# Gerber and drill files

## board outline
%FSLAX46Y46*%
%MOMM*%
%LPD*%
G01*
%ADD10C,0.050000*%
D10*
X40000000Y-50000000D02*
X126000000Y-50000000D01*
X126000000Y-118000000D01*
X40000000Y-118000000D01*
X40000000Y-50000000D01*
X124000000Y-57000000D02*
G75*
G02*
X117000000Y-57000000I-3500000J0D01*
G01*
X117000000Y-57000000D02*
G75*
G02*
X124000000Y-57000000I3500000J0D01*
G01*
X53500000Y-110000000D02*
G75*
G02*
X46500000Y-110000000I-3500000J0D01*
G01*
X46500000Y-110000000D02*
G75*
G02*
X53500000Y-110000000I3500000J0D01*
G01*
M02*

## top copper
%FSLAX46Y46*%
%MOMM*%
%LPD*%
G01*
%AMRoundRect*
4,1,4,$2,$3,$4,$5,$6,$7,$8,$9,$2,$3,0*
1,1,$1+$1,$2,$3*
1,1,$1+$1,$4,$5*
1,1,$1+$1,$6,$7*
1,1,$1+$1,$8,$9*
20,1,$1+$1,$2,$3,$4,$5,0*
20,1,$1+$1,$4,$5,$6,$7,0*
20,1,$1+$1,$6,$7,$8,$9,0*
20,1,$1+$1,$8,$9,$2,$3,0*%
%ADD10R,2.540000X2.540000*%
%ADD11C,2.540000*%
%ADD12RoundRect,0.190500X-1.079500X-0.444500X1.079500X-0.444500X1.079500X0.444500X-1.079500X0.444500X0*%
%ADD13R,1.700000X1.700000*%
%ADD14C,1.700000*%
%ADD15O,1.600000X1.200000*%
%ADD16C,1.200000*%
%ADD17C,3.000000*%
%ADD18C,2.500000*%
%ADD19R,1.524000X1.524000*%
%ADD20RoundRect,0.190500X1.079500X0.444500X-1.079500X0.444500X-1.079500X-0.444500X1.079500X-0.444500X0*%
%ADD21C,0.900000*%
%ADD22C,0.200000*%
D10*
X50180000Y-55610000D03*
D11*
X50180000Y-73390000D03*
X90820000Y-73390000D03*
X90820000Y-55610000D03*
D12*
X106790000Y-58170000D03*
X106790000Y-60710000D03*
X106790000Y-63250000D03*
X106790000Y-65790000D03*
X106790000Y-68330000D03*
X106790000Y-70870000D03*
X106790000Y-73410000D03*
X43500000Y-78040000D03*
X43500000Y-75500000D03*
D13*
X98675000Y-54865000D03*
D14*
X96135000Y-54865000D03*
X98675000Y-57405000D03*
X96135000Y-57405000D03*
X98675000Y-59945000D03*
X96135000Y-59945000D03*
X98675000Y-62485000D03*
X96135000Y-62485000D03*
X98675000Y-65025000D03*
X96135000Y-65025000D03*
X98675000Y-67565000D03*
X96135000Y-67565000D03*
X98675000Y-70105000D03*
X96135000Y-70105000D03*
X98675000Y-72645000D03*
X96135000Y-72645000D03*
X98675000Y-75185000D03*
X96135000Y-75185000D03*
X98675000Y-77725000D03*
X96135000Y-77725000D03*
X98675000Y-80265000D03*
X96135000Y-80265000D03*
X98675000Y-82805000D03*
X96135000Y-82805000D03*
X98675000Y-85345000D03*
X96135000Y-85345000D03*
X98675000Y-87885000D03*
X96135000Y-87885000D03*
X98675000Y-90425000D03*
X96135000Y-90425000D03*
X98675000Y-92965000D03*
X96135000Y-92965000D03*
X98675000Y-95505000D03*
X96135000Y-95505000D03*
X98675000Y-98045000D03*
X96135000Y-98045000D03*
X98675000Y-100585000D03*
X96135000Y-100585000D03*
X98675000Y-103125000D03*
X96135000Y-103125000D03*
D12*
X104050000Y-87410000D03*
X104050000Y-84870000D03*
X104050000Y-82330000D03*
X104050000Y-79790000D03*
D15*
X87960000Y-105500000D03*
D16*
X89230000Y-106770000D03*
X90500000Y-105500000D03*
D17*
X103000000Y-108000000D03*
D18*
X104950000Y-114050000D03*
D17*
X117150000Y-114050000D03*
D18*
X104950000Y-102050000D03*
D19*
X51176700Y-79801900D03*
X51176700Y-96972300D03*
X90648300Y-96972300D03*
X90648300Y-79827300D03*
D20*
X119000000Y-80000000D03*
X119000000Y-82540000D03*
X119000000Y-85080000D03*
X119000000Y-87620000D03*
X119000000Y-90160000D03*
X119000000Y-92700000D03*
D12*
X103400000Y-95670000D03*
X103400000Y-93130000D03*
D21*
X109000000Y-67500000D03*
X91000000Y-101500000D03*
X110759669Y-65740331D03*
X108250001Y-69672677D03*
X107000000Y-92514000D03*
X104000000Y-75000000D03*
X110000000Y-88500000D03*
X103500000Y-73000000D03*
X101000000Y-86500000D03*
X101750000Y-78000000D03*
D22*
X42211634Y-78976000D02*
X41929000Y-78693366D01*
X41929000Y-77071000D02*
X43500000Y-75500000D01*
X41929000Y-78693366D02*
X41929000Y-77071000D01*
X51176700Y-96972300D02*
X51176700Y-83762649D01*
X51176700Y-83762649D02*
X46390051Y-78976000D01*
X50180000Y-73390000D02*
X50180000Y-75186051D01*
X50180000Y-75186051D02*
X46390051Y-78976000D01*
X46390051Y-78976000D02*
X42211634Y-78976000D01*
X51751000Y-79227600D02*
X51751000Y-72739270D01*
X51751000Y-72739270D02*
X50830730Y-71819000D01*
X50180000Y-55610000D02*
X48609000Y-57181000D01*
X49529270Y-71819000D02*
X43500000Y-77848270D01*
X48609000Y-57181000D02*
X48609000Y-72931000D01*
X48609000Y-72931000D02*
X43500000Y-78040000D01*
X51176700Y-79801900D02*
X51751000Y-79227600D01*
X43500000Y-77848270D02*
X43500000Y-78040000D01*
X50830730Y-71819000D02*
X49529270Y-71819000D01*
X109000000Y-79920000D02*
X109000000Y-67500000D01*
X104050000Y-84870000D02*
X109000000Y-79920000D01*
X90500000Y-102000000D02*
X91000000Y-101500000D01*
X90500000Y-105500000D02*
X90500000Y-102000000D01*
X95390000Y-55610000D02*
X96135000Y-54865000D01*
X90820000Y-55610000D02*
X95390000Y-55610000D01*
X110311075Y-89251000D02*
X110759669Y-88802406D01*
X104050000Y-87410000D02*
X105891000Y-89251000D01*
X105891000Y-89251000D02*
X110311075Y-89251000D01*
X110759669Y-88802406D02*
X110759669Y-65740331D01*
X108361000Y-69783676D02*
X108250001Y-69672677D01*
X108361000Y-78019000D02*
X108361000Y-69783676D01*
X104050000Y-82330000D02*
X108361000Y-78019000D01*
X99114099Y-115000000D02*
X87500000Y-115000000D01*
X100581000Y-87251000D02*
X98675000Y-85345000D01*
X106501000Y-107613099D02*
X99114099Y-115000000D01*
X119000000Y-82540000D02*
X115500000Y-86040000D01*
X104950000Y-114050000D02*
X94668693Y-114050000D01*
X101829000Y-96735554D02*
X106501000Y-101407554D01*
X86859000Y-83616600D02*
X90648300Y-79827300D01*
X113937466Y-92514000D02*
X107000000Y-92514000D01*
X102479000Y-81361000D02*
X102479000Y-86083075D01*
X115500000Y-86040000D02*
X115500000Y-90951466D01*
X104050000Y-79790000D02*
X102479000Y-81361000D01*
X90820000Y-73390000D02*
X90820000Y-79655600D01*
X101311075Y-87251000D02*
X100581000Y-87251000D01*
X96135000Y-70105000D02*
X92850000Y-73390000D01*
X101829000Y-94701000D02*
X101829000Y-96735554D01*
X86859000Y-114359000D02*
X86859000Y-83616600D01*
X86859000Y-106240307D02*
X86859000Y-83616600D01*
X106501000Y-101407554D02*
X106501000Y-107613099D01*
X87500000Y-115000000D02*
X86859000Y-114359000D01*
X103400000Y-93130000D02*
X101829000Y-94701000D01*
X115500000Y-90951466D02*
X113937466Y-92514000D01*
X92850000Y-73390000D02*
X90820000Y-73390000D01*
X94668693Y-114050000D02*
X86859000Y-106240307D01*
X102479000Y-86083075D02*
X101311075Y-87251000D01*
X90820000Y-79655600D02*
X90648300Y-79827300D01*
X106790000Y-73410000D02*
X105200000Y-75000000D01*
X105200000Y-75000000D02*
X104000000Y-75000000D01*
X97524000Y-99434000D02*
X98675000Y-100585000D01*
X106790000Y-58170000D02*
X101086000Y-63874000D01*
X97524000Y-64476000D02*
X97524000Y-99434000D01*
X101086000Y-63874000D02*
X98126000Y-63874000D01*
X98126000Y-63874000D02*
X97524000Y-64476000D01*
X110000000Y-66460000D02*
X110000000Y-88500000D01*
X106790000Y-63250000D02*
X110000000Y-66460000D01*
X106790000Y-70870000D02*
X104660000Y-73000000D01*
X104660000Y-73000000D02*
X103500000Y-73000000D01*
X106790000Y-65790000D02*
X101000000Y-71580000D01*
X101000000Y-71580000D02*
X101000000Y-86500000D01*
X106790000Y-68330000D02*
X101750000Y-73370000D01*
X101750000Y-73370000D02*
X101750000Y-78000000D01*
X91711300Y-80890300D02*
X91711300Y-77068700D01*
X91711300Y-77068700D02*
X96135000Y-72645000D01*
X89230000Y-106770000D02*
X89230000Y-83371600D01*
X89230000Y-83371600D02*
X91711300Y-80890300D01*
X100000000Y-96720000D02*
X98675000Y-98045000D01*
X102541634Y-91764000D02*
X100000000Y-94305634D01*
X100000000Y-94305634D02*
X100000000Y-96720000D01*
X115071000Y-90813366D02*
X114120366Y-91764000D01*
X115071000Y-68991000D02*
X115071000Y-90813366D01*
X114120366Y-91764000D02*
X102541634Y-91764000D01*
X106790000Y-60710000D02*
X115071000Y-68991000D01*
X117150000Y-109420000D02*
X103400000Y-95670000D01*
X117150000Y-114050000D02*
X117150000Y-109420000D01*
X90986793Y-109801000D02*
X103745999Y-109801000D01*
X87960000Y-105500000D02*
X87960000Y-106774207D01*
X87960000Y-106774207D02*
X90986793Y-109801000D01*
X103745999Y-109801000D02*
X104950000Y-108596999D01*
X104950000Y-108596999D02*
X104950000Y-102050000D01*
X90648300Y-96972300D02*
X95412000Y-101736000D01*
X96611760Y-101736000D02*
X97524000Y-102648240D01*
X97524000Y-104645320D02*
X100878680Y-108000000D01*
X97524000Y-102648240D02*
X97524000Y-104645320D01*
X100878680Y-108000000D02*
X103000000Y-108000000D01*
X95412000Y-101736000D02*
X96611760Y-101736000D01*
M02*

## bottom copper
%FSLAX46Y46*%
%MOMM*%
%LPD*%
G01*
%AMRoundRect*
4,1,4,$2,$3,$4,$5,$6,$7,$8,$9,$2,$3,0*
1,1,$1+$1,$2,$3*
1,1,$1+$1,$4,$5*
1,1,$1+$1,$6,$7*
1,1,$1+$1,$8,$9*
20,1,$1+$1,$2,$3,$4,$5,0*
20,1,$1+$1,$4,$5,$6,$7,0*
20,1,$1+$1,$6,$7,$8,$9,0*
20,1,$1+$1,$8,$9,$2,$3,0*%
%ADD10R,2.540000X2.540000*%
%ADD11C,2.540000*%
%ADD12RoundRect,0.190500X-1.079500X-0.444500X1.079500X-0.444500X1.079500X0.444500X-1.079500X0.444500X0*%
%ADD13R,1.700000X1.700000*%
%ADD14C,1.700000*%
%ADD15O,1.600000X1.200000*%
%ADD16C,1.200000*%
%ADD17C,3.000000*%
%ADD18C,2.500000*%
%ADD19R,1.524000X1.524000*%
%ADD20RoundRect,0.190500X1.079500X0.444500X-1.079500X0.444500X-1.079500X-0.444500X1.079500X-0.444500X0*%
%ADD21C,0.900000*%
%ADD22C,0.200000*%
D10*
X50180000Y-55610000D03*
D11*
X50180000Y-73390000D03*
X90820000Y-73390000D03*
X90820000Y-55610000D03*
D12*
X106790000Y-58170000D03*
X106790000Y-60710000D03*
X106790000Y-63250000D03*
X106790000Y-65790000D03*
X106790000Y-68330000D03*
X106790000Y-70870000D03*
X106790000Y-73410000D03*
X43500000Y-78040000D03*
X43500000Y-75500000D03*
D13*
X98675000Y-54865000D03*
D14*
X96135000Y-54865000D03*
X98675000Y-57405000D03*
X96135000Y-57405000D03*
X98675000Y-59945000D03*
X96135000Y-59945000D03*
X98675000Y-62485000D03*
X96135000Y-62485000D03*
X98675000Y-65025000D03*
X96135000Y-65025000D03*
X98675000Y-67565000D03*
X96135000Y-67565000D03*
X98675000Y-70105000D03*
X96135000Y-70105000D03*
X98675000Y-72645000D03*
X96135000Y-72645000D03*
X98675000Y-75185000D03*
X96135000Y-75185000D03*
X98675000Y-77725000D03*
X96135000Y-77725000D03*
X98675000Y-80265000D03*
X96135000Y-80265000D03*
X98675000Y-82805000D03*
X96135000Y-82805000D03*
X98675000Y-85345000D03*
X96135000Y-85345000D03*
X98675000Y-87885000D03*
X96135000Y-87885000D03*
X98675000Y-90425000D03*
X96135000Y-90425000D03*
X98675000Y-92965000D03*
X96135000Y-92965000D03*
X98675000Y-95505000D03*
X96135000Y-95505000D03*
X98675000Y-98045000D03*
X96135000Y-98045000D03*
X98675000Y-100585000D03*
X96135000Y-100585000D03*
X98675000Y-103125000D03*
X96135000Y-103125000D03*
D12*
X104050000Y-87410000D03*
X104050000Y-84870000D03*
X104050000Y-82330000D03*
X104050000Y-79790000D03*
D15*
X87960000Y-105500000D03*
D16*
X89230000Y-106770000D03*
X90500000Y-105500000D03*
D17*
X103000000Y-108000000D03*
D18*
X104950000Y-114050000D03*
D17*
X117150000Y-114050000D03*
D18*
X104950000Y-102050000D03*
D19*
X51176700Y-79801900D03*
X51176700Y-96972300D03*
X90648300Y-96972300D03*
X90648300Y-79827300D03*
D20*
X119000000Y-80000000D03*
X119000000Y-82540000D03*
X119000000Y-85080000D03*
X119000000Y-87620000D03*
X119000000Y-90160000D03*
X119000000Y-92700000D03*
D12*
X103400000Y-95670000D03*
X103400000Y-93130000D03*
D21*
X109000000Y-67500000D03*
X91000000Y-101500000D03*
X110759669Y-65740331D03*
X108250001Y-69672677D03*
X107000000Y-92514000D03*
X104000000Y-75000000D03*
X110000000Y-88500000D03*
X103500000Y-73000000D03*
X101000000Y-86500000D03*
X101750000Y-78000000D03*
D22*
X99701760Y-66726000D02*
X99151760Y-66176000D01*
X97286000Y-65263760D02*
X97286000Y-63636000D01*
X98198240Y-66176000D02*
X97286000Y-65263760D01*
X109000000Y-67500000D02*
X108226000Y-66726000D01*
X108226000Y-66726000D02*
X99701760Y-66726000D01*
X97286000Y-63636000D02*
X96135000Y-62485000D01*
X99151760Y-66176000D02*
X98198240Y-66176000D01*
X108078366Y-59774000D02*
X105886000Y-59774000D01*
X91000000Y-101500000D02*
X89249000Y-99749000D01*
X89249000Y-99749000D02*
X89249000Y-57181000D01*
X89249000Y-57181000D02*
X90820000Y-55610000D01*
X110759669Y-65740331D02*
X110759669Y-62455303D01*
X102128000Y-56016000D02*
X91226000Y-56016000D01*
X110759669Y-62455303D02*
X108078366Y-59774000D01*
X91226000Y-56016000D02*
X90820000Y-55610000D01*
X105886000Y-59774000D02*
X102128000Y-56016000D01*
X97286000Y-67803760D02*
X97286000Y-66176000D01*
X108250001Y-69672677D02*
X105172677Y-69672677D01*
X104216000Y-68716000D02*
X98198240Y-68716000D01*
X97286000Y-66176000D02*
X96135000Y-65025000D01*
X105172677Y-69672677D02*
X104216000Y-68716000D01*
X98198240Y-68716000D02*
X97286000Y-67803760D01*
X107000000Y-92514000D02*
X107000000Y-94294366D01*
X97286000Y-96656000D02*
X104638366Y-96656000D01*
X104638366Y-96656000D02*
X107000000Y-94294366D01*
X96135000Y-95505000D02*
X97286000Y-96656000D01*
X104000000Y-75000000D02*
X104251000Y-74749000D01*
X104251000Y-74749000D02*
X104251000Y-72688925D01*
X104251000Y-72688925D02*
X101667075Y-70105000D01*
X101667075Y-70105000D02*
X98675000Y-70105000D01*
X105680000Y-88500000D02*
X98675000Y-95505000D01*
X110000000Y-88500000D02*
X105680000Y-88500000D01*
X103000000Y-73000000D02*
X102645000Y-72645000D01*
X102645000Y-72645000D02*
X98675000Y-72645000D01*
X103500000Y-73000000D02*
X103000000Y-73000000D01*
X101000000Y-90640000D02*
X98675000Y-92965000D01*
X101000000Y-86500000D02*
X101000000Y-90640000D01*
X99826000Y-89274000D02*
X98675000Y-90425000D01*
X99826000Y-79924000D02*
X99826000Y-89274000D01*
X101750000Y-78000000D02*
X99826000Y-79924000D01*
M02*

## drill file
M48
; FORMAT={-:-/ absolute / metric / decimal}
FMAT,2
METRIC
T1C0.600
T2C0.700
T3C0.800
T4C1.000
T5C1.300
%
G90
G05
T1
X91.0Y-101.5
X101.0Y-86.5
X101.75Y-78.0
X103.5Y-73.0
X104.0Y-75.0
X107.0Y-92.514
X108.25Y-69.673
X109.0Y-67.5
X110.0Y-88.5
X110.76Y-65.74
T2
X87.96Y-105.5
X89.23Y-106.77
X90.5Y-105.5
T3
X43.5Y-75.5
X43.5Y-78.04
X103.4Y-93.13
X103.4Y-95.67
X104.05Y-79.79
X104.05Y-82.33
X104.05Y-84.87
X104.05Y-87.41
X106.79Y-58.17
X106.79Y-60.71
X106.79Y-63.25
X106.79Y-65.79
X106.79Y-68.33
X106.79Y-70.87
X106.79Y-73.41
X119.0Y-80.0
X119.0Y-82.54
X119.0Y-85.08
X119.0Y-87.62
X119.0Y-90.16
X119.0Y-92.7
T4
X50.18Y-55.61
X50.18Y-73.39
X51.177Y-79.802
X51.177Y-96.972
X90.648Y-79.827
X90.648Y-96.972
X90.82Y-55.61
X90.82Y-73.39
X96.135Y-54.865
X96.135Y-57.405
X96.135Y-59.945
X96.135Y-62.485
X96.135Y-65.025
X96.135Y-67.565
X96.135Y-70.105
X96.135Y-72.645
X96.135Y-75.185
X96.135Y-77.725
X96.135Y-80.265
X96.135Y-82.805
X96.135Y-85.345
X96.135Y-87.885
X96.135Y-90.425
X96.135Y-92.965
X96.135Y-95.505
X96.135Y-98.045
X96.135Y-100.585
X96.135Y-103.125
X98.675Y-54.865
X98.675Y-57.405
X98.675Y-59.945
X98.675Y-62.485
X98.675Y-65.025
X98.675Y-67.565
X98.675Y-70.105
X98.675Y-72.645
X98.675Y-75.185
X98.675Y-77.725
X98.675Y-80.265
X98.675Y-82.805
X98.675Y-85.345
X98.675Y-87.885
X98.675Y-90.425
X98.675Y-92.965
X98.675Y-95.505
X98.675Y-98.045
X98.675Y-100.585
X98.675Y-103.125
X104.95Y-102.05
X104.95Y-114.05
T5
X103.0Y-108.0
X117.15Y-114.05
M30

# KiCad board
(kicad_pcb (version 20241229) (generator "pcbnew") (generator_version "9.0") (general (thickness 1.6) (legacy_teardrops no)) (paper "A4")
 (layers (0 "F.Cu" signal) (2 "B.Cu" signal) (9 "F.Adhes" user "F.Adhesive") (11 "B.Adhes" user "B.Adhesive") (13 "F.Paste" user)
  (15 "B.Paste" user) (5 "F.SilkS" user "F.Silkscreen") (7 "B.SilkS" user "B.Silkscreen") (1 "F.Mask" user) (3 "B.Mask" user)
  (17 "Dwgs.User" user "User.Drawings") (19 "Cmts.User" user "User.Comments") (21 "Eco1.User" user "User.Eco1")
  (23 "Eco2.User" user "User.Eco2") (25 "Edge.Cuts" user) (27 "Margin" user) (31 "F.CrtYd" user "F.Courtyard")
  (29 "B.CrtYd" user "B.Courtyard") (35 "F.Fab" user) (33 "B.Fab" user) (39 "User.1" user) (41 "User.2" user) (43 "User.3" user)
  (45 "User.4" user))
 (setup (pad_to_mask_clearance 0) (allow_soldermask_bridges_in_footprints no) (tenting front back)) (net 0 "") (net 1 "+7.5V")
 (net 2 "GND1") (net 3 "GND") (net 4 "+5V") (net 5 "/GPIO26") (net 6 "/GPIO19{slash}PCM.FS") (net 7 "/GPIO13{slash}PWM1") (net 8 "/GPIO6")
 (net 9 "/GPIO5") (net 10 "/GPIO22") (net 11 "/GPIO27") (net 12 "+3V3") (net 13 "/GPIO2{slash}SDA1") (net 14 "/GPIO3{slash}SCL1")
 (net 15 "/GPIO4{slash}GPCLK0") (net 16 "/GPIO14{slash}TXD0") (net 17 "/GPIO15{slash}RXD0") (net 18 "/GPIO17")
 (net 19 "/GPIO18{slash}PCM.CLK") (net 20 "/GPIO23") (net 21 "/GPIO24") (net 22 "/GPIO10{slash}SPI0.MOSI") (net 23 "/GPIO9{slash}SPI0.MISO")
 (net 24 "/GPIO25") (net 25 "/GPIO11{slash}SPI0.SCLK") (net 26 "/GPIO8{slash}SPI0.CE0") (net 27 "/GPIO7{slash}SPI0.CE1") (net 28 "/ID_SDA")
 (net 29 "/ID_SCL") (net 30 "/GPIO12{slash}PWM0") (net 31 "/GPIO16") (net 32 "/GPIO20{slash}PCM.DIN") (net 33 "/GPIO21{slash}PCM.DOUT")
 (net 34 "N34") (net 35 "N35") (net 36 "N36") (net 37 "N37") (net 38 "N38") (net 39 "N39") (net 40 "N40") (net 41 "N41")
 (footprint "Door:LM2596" (layer "F.Cu") (at 50.18 55.61)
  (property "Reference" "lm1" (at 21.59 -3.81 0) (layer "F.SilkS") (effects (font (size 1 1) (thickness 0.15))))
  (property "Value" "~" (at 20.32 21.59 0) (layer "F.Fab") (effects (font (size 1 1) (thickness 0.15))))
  (pad "1" thru_hole rect (at 0 0) (size 2.54 2.54) (drill 1) (layers "*.Cu" "*.Mask") (remove_unused_layers no) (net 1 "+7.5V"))
  (pad "2" thru_hole circle (at 0 17.78) (size 2.54 2.54) (drill 1) (layers "*.Cu" "*.Mask") (remove_unused_layers no) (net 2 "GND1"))
  (pad "3" thru_hole circle (at 40.64 17.78) (size 2.54 2.54) (drill 1) (layers "*.Cu" "*.Mask") (remove_unused_layers no) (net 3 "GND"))
  (pad "4" thru_hole circle (at 40.64 0) (size 2.54 2.54) (drill 1) (layers "*.Cu" "*.Mask") (remove_unused_layers no) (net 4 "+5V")))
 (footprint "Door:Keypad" (layer "F.Cu") (at 101.71 75.95)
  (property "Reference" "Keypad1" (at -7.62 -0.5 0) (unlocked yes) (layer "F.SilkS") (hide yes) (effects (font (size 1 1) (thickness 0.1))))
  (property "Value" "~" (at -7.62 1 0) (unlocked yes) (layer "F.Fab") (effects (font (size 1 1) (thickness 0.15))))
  (pad "2" thru_hole roundrect (at 5.08 -17.78) (size 2.54 1.27) (drill 0.8) (layers "*.Cu" "*.Mask") (remove_unused_layers no)
   (roundrect_rratio 0.15) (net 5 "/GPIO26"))
  (pad "3" thru_hole roundrect (at 5.08 -15.24) (size 2.54 1.27) (drill 0.8) (layers "*.Cu" "*.Mask") (remove_unused_layers no)
   (roundrect_rratio 0.15) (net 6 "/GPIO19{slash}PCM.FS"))
  (pad "4" thru_hole roundrect (at 5.08 -12.7) (size 2.54 1.27) (drill 0.8) (layers "*.Cu" "*.Mask") (remove_unused_layers no)
   (roundrect_rratio 0.15) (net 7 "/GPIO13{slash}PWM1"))
  (pad "5" thru_hole roundrect (at 5.08 -10.16) (size 2.54 1.27) (drill 0.8) (layers "*.Cu" "*.Mask") (remove_unused_layers no)
   (roundrect_rratio 0.15) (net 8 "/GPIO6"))
  (pad "6" thru_hole roundrect (at 5.08 -7.62) (size 2.54 1.27) (drill 0.8) (layers "*.Cu" "*.Mask") (remove_unused_layers no)
   (roundrect_rratio 0.15) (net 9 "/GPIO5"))
  (pad "7" thru_hole roundrect (at 5.08 -5.08) (size 2.54 1.27) (drill 0.8) (layers "*.Cu" "*.Mask") (remove_unused_layers no)
   (roundrect_rratio 0.15) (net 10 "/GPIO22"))
  (pad "8" thru_hole roundrect (at 5.08 -2.54) (size 2.54 1.27) (drill 0.8) (layers "*.Cu" "*.Mask") (remove_unused_layers no)
   (roundrect_rratio 0.15) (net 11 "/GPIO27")))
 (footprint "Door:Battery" (layer "F.Cu") (at 48.58 83.12)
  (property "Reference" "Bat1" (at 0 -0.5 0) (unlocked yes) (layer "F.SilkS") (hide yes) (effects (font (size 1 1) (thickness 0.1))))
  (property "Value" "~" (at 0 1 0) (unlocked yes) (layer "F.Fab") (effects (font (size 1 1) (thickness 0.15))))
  (pad "1" thru_hole roundrect (at -5.08 -5.08) (size 2.54 1.27) (drill 0.8) (layers "*.Cu" "*.Mask") (remove_unused_layers no)
   (roundrect_rratio 0.15) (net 1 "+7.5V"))
  (pad "2" thru_hole roundrect (at -5.08 -7.62) (size 2.54 1.27) (drill 0.8) (layers "*.Cu" "*.Mask") (remove_unused_layers no)
   (roundrect_rratio 0.15) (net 2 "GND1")))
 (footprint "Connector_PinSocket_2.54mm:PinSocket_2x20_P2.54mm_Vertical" (layer "F.Cu") (at 98.675 54.865)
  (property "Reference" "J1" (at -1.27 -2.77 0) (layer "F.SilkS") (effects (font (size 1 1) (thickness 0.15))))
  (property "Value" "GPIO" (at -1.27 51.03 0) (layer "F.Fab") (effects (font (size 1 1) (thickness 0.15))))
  (pad "1" thru_hole rect (at 0 0) (size 1.7 1.7) (drill 1) (layers "*.Cu" "*.Mask") (remove_unused_layers no) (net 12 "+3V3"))
  (pad "2" thru_hole circle (at -2.54 0) (size 1.7 1.7) (drill 1) (layers "*.Cu" "*.Mask") (remove_unused_layers no) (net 4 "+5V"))
  (pad "3" thru_hole circle (at 0 2.54) (size 1.7 1.7) (drill 1) (layers "*.Cu" "*.Mask") (remove_unused_layers no)
   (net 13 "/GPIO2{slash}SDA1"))
  (pad "4" thru_hole circle (at -2.54 2.54) (size 1.7 1.7) (drill 1) (layers "*.Cu" "*.Mask") (remove_unused_layers no) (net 4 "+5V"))
  (pad "5" thru_hole circle (at 0 5.08) (size 1.7 1.7) (drill 1) (layers "*.Cu" "*.Mask") (remove_unused_layers no)
   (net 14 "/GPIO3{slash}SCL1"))
  (pad "6" thru_hole circle (at -2.54 5.08) (size 1.7 1.7) (drill 1) (layers "*.Cu" "*.Mask") (remove_unused_layers no) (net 3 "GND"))
  (pad "7" thru_hole circle (at 0 7.62) (size 1.7 1.7) (drill 1) (layers "*.Cu" "*.Mask") (remove_unused_layers no)
   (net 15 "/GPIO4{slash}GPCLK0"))
  (pad "8" thru_hole circle (at -2.54 7.62) (size 1.7 1.7) (drill 1) (layers "*.Cu" "*.Mask") (remove_unused_layers no)
   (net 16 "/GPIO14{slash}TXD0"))
  (pad "9" thru_hole circle (at 0 10.16) (size 1.7 1.7) (drill 1) (layers "*.Cu" "*.Mask") (remove_unused_layers no) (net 3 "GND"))
  (pad "10" thru_hole circle (at -2.54 10.16) (size 1.7 1.7) (drill 1) (layers "*.Cu" "*.Mask") (remove_unused_layers no)
   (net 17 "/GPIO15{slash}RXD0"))
  (pad "11" thru_hole circle (at 0 12.7) (size 1.7 1.7) (drill 1) (layers "*.Cu" "*.Mask") (remove_unused_layers no) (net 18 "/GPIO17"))
  (pad "12" thru_hole circle (at -2.54 12.7) (size 1.7 1.7) (drill 1) (layers "*.Cu" "*.Mask") (remove_unused_layers no)
   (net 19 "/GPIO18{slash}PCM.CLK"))
  (pad "13" thru_hole circle (at 0 15.24) (size 1.7 1.7) (drill 1) (layers "*.Cu" "*.Mask") (remove_unused_layers no) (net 11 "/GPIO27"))
  (pad "14" thru_hole circle (at -2.54 15.24) (size 1.7 1.7) (drill 1) (layers "*.Cu" "*.Mask") (remove_unused_layers no) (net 3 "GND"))
  (pad "15" thru_hole circle (at 0 17.78) (size 1.7 1.7) (drill 1) (layers "*.Cu" "*.Mask") (remove_unused_layers no) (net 10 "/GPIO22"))
  (pad "16" thru_hole circle (at -2.54 17.78) (size 1.7 1.7) (drill 1) (layers "*.Cu" "*.Mask") (remove_unused_layers no) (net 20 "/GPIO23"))
  (pad "17" thru_hole circle (at 0 20.32) (size 1.7 1.7) (drill 1) (layers "*.Cu" "*.Mask") (remove_unused_layers no) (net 12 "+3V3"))
  (pad "18" thru_hole circle (at -2.54 20.32) (size 1.7 1.7) (drill 1) (layers "*.Cu" "*.Mask") (remove_unused_layers no) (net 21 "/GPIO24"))
  (pad "19" thru_hole circle (at 0 22.86) (size 1.7 1.7) (drill 1) (layers "*.Cu" "*.Mask") (remove_unused_layers no)
   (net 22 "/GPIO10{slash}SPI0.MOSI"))
  (pad "20" thru_hole circle (at -2.54 22.86) (size 1.7 1.7) (drill 1) (layers "*.Cu" "*.Mask") (remove_unused_layers no) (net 3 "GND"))
  (pad "21" thru_hole circle (at 0 25.4) (size 1.7 1.7) (drill 1) (layers "*.Cu" "*.Mask") (remove_unused_layers no)
   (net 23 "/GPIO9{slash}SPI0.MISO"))
  (pad "22" thru_hole circle (at -2.54 25.4) (size 1.7 1.7) (drill 1) (layers "*.Cu" "*.Mask") (remove_unused_layers no) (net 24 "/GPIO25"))
  (pad "23" thru_hole circle (at 0 27.94) (size 1.7 1.7) (drill 1) (layers "*.Cu" "*.Mask") (remove_unused_layers no)
   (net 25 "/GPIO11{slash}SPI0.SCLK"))
  (pad "24" thru_hole circle (at -2.54 27.94) (size 1.7 1.7) (drill 1) (layers "*.Cu" "*.Mask") (remove_unused_layers no)
   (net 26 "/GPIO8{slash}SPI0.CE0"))
  (pad "25" thru_hole circle (at 0 30.48) (size 1.7 1.7) (drill 1) (layers "*.Cu" "*.Mask") (remove_unused_layers no) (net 3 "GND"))
  (pad "26" thru_hole circle (at -2.54 30.48) (size 1.7 1.7) (drill 1) (layers "*.Cu" "*.Mask") (remove_unused_layers no)
   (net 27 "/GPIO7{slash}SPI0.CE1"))
  (pad "27" thru_hole circle (at 0 33.02) (size 1.7 1.7) (drill 1) (layers "*.Cu" "*.Mask") (remove_unused_layers no) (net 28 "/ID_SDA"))
  (pad "28" thru_hole circle (at -2.54 33.02) (size 1.7 1.7) (drill 1) (layers "*.Cu" "*.Mask") (remove_unused_layers no) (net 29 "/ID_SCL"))
  (pad "29" thru_hole circle (at 0 35.56) (size 1.7 1.7) (drill 1) (layers "*.Cu" "*.Mask") (remove_unused_layers no) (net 9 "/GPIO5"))
  (pad "30" thru_hole circle (at -2.54 35.56) (size 1.7 1.7) (drill 1) (layers "*.Cu" "*.Mask") (remove_unused_layers no) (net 3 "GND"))
  (pad "31" thru_hole circle (at 0 38.1) (size 1.7 1.7) (drill 1) (layers "*.Cu" "*.Mask") (remove_unused_layers no) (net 8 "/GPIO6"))
  (pad "32" thru_hole circle (at -2.54 38.1) (size 1.7 1.7) (drill 1) (layers "*.Cu" "*.Mask") (remove_unused_layers no)
   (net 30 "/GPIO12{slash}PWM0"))
  (pad "33" thru_hole circle (at 0 40.64) (size 1.7 1.7) (drill 1) (layers "*.Cu" "*.Mask") (remove_unused_layers no)
   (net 7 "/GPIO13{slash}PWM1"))
  (pad "34" thru_hole circle (at -2.54 40.64) (size 1.7 1.7) (drill 1) (layers "*.Cu" "*.Mask") (remove_unused_layers no) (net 3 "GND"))
  (pad "35" thru_hole circle (at 0 43.18) (size 1.7 1.7) (drill 1) (layers "*.Cu" "*.Mask") (remove_unused_layers no)
   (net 6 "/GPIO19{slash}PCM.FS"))
  (pad "36" thru_hole circle (at -2.54 43.18) (size 1.7 1.7) (drill 1) (layers "*.Cu" "*.Mask") (remove_unused_layers no) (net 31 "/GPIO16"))
  (pad "37" thru_hole circle (at 0 45.72) (size 1.7 1.7) (drill 1) (layers "*.Cu" "*.Mask") (remove_unused_layers no) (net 5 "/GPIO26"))
  (pad "38" thru_hole circle (at -2.54 45.72) (size 1.7 1.7) (drill 1) (layers "*.Cu" "*.Mask") (remove_unused_layers no)
   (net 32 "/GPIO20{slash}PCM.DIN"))
  (pad "39" thru_hole circle (at 0 48.26) (size 1.7 1.7) (drill 1) (layers "*.Cu" "*.Mask") (remove_unused_layers no) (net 3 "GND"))
  (pad "40" thru_hole circle (at -2.54 48.26) (size 1.7 1.7) (drill 1) (layers "*.Cu" "*.Mask") (remove_unused_layers no)
   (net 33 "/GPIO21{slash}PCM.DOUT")))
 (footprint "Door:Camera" (layer "F.Cu") (at 106.59 97.57)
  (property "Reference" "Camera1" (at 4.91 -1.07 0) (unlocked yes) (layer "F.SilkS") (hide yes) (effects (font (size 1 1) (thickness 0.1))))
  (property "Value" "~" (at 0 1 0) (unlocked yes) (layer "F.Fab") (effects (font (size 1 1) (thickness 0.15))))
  (pad "1" thru_hole roundrect (at -2.54 -10.16) (size 2.54 1.27) (drill 0.8) (layers "*.Cu" "*.Mask") (remove_unused_layers no)
   (roundrect_rratio 0.15) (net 4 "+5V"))
  (pad "2" thru_hole roundrect (at -2.54 -12.7) (size 2.54 1.27) (drill 0.8) (layers "*.Cu" "*.Mask") (remove_unused_layers no)
   (roundrect_rratio 0.15) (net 16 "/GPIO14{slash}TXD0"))
  (pad "3" thru_hole roundrect (at -2.54 -15.24) (size 2.54 1.27) (drill 0.8) (layers "*.Cu" "*.Mask") (remove_unused_layers no)
   (roundrect_rratio 0.15) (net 17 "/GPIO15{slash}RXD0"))
  (pad "4" thru_hole roundrect (at -2.54 -17.78) (size 2.54 1.27) (drill 0.8) (layers "*.Cu" "*.Mask") (remove_unused_layers no)
   (roundrect_rratio 0.15) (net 3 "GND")))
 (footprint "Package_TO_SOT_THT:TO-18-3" (layer "F.Cu") (at 87.96 105.5)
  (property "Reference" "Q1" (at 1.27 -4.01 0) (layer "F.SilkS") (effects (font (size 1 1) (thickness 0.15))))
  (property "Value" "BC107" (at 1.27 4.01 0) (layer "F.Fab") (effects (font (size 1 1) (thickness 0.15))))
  (pad "1" thru_hole oval (at 0 0) (size 1.6 1.2) (drill 0.7) (layers "*.Cu" "*.Mask") (remove_unused_layers no) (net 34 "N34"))
  (pad "2" thru_hole circle (at 1.27 1.27) (size 1.2 1.2) (drill 0.7) (layers "*.Cu" "*.Mask") (remove_unused_layers no) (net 20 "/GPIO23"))
  (pad "3" thru_hole circle (at 2.54 0) (size 1.2 1.2) (drill 0.7) (layers "*.Cu" "*.Mask") (remove_unused_layers no) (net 4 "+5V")))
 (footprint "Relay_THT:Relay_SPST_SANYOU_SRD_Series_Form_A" (layer "F.Cu") (at 103 108)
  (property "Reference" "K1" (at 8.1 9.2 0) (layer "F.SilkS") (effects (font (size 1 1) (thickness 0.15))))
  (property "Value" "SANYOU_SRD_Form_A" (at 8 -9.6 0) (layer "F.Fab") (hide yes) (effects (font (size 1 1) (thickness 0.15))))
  (pad "1" thru_hole circle (at 0 0 90) (size 3 3) (drill 1.3) (layers "*.Cu" "*.Mask") (remove_unused_layers no) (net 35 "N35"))
  (pad "2" thru_hole circle (at 1.95 6.05 90) (size 2.5 2.5) (drill 1) (layers "*.Cu" "*.Mask") (remove_unused_layers no) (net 3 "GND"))
  (pad "3" thru_hole circle (at 14.15 6.05 90) (size 3 3) (drill 1.3) (layers "*.Cu" "*.Mask") (remove_unused_layers no) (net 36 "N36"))
  (pad "5" thru_hole circle (at 1.95 -5.95 90) (size 2.5 2.5) (drill 1) (layers "*.Cu" "*.Mask") (remove_unused_layers no) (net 34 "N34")))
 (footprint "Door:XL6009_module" (layer "F.Cu") (at 92.5025 98.9535)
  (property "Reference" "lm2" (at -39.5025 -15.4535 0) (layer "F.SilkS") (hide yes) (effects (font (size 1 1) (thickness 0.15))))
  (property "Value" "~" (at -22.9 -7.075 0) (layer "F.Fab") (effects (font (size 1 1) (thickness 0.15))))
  (pad "1" thru_hole rect (at -41.3258 -19.1516) (size 1.524 1.524) (drill 1) (layers "*.Cu" "*.Mask") (remove_unused_layers no)
   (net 1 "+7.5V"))
  (pad "2" thru_hole rect (at -41.3258 -1.9812) (size 1.524 1.524) (drill 1) (layers "*.Cu" "*.Mask") (remove_unused_layers no)
   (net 2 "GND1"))
  (pad "3" thru_hole rect (at -1.8542 -1.9812) (size 1.524 1.524) (drill 1) (layers "*.Cu" "*.Mask") (remove_unused_layers no)
   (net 35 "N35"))
  (pad "4" thru_hole rect (at -1.8542 -19.1262) (size 1.524 1.524) (drill 1) (layers "*.Cu" "*.Mask") (remove_unused_layers no)
   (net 3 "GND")))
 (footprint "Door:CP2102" (layer "F.Cu") (at 116.46 77.46 180)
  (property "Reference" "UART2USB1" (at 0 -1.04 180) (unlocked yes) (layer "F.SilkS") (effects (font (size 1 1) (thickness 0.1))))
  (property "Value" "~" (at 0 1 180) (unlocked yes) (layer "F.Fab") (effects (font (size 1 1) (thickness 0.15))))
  (pad "1" thru_hole roundrect (at -2.54 -2.54 180) (size 2.54 1.27) (drill 0.8) (layers "*.Cu" "*.Mask") (remove_unused_layers no)
   (roundrect_rratio 0.15) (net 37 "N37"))
  (pad "2" thru_hole roundrect (at -2.54 -5.08 180) (size 2.54 1.27) (drill 0.8) (layers "*.Cu" "*.Mask") (remove_unused_layers no)
   (roundrect_rratio 0.15) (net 3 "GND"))
  (pad "3" thru_hole roundrect (at -2.54 -7.62 180) (size 2.54 1.27) (drill 0.8) (layers "*.Cu" "*.Mask") (remove_unused_layers no)
   (roundrect_rratio 0.15) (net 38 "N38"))
  (pad "4" thru_hole roundrect (at -2.54 -10.16 180) (size 2.54 1.27) (drill 0.8) (layers "*.Cu" "*.Mask") (remove_unused_layers no)
   (roundrect_rratio 0.15) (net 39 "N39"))
  (pad "5" thru_hole roundrect (at -2.54 -12.7 180) (size 2.54 1.27) (drill 0.8) (layers "*.Cu" "*.Mask") (remove_unused_layers no)
   (roundrect_rratio 0.15) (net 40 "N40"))
  (pad "6" thru_hole roundrect (at -2.54 -15.24 180) (size 2.54 1.27) (drill 0.8) (layers "*.Cu" "*.Mask") (remove_unused_layers no)
   (roundrect_rratio 0.15) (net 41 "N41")))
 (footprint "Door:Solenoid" (layer "F.Cu") (at 105.94 98.21)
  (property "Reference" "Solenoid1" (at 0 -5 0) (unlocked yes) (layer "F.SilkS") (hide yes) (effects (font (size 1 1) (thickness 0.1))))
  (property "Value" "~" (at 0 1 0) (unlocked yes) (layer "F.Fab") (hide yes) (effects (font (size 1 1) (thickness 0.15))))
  (pad "1" thru_hole roundrect (at -2.54 -2.54) (size 2.54 1.27) (drill 0.8) (layers "*.Cu" "*.Mask") (remove_unused_layers no)
   (roundrect_rratio 0.15) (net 36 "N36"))
  (pad "2" thru_hole roundrect (at -2.54 -5.08) (size 2.54 1.27) (drill 0.8) (layers "*.Cu" "*.Mask") (remove_unused_layers no)
   (roundrect_rratio 0.15) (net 3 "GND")))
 (gr_rect (start 40 50) (end 126 118) (stroke (width 0.05) (type default)) (fill no) (layer "Edge.Cuts"))
 (gr_circle (center 120.5 57) (end 124 57) (stroke (width 0.05) (type default)) (fill no) (layer "Edge.Cuts"))
 (gr_circle (center 50 110) (end 53.5 110) (stroke (width 0.05) (type default)) (fill no) (layer "Edge.Cuts"))
 (segment (start 42.211634 78.976) (end 41.929 78.693366) (width 0.2) (layer "F.Cu") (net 2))
 (segment (start 41.929 77.071) (end 43.5 75.5) (width 0.2) (layer "F.Cu") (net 2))
 (segment (start 41.929 78.693366) (end 41.929 77.071) (width 0.2) (layer "F.Cu") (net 2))
 (segment (start 51.1767 96.9723) (end 51.1767 83.762649) (width 0.2) (layer "F.Cu") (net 2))
 (segment (start 51.1767 83.762649) (end 46.390051 78.976) (width 0.2) (layer "F.Cu") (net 2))
 (segment (start 50.18 73.39) (end 50.18 75.186051) (width 0.2) (layer "F.Cu") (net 2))
 (segment (start 50.18 75.186051) (end 46.390051 78.976) (width 0.2) (layer "F.Cu") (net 2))
 (segment (start 46.390051 78.976) (end 42.211634 78.976) (width 0.2) (layer "F.Cu") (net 2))
 (segment (start 51.751 79.2276) (end 51.751 72.73927) (width 0.2) (layer "F.Cu") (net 1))
 (segment (start 51.751 72.73927) (end 50.83073 71.819) (width 0.2) (layer "F.Cu") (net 1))
 (segment (start 50.18 55.61) (end 48.609 57.181) (width 0.2) (layer "F.Cu") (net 1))
 (segment (start 49.52927 71.819) (end 43.5 77.84827) (width 0.2) (layer "F.Cu") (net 1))
 (segment (start 48.609 57.181) (end 48.609 72.931) (width 0.2) (layer "F.Cu") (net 1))
 (segment (start 48.609 72.931) (end 43.5 78.04) (width 0.2) (layer "F.Cu") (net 1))
 (segment (start 51.1767 79.8019) (end 51.751 79.2276) (width 0.2) (layer "F.Cu") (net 1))
 (segment (start 43.5 77.84827) (end 43.5 78.04) (width 0.2) (layer "F.Cu") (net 1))
 (segment (start 50.83073 71.819) (end 49.52927 71.819) (width 0.2) (layer "F.Cu") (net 1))
 (segment (start 109 79.92) (end 109 67.5) (width 0.2) (layer "F.Cu") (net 16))
 (segment (start 104.05 84.87) (end 109 79.92) (width 0.2) (layer "F.Cu") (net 16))
 (via (at 109 67.5) (size 0.9) (drill 0.6) (layers "F.Cu" "B.Cu") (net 16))
 (segment (start 99.70176 66.726) (end 99.15176 66.176) (width 0.2) (layer "B.Cu") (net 16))
 (segment (start 97.286 65.26376) (end 97.286 63.636) (width 0.2) (layer "B.Cu") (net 16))
 (segment (start 98.19824 66.176) (end 97.286 65.26376) (width 0.2) (layer "B.Cu") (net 16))
 (segment (start 109 67.5) (end 108.226 66.726) (width 0.2) (layer "B.Cu") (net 16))
 (segment (start 108.226 66.726) (end 99.70176 66.726) (width 0.2) (layer "B.Cu") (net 16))
 (segment (start 97.286 63.636) (end 96.135 62.485) (width 0.2) (layer "B.Cu") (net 16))
 (segment (start 99.15176 66.176) (end 98.19824 66.176) (width 0.2) (layer "B.Cu") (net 16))
 (segment (start 90.5 102) (end 91 101.5) (width 0.2) (layer "F.Cu") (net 4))
 (segment (start 90.5 105.5) (end 90.5 102) (width 0.2) (layer "F.Cu") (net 4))
 (segment (start 95.39 55.61) (end 96.135 54.865) (width 0.2) (layer "F.Cu") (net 4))
 (segment (start 90.82 55.61) (end 95.39 55.61) (width 0.2) (layer "F.Cu") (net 4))
 (segment (start 110.311075 89.251) (end 110.759669 88.802406) (width 0.2) (layer "F.Cu") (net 4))
 (segment (start 104.05 87.41) (end 105.891 89.251) (width 0.2) (layer "F.Cu") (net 4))
 (segment (start 105.891 89.251) (end 110.311075 89.251) (width 0.2) (layer "F.Cu") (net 4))
 (segment (start 110.759669 88.802406) (end 110.759669 65.740331) (width 0.2) (layer "F.Cu") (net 4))
 (via (at 91 101.5) (size 0.9) (drill 0.6) (layers "F.Cu" "B.Cu") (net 4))
 (via (at 110.759669 65.740331) (size 0.9) (drill 0.6) (layers "F.Cu" "B.Cu") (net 4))
 (segment (start 108.078366 59.774) (end 105.886 59.774) (width 0.2) (layer "B.Cu") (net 4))
 (segment (start 91 101.5) (end 89.249 99.749) (width 0.2) (layer "B.Cu") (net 4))
 (segment (start 89.249 99.749) (end 89.249 57.181) (width 0.2) (layer "B.Cu") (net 4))
 (segment (start 89.249 57.181) (end 90.82 55.61) (width 0.2) (layer "B.Cu") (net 4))
 (segment (start 110.759669 65.740331) (end 110.759669 62.455303) (width 0.2) (layer "B.Cu") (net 4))
 (segment (start 102.128 56.016) (end 91.226 56.016) (width 0.2) (layer "B.Cu") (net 4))
 (segment (start 110.759669 62.455303) (end 108.078366 59.774) (width 0.2) (layer "B.Cu") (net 4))
 (segment (start 91.226 56.016) (end 90.82 55.61) (width 0.2) (layer "B.Cu") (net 4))
 (segment (start 105.886 59.774) (end 102.128 56.016) (width 0.2) (layer "B.Cu") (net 4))
 (segment (start 108.361 69.783676) (end 108.250001 69.672677) (width 0.2) (layer "F.Cu") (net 17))
 (segment (start 108.361 78.019) (end 108.361 69.783676) (width 0.2) (layer "F.Cu") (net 17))
 (segment (start 104.05 82.33) (end 108.361 78.019) (width 0.2) (layer "F.Cu") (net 17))
 (via (at 108.250001 69.672677) (size 0.9) (drill 0.6) (layers "F.Cu" "B.Cu") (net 17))
 (segment (start 97.286 67.80376) (end 97.286 66.176) (width 0.2) (layer "B.Cu") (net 17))
 (segment (start 108.250001 69.672677) (end 105.172677 69.672677) (width 0.2) (layer "B.Cu") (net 17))
 (segment (start 104.216 68.716) (end 98.19824 68.716) (width 0.2) (layer "B.Cu") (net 17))
 (segment (start 97.286 66.176) (end 96.135 65.025) (width 0.2) (layer "B.Cu") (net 17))
 (segment (start 105.172677 69.672677) (end 104.216 68.716) (width 0.2) (layer "B.Cu") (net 17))
 (segment (start 98.19824 68.716) (end 97.286 67.80376) (width 0.2) (layer "B.Cu") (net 17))
 (segment (start 99.114099 115) (end 87.5 115) (width 0.2) (layer "F.Cu") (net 3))
 (segment (start 100.581 87.251) (end 98.675 85.345) (width 0.2) (layer "F.Cu") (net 3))
 (segment (start 106.501 107.613099) (end 99.114099 115) (width 0.2) (layer "F.Cu") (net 3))
 (segment (start 119 82.54) (end 115.5 86.04) (width 0.2) (layer "F.Cu") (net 3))
 (segment (start 104.95 114.05) (end 94.668693 114.05) (width 0.2) (layer "F.Cu") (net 3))
 (segment (start 101.829 96.735554) (end 106.501 101.407554) (width 0.2) (layer "F.Cu") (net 3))
 (segment (start 86.859 83.6166) (end 90.6483 79.8273) (width 0.2) (layer "F.Cu") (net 3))
 (segment (start 113.937466 92.514) (end 107 92.514) (width 0.2) (layer "F.Cu") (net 3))
 (segment (start 102.479 81.361) (end 102.479 86.083075) (width 0.2) (layer "F.Cu") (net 3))
 (segment (start 115.5 86.04) (end 115.5 90.951466) (width 0.2) (layer "F.Cu") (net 3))
 (segment (start 104.05 79.79) (end 102.479 81.361) (width 0.2) (layer "F.Cu") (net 3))
 (segment (start 90.82 73.39) (end 90.82 79.6556) (width 0.2) (layer "F.Cu") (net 3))
 (segment (start 101.311075 87.251) (end 100.581 87.251) (width 0.2) (layer "F.Cu") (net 3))
 (segment (start 96.135 70.105) (end 92.85 73.39) (width 0.2) (layer "F.Cu") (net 3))
 (segment (start 101.829 94.701) (end 101.829 96.735554) (width 0.2) (layer "F.Cu") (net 3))
 (segment (start 86.859 114.359) (end 86.859 83.6166) (width 0.2) (layer "F.Cu") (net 3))
 (segment (start 86.859 106.240307) (end 86.859 83.6166) (width 0.2) (layer "F.Cu") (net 3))
 (segment (start 106.501 101.407554) (end 106.501 107.613099) (width 0.2) (layer "F.Cu") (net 3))
 (segment (start 87.5 115) (end 86.859 114.359) (width 0.2) (layer "F.Cu") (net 3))
 (segment (start 103.4 93.13) (end 101.829 94.701) (width 0.2) (layer "F.Cu") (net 3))
 (segment (start 115.5 90.951466) (end 113.937466 92.514) (width 0.2) (layer "F.Cu") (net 3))
 (segment (start 92.85 73.39) (end 90.82 73.39) (width 0.2) (layer "F.Cu") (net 3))
 (segment (start 94.668693 114.05) (end 86.859 106.240307) (width 0.2) (layer "F.Cu") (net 3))
 (segment (start 102.479 86.083075) (end 101.311075 87.251) (width 0.2) (layer "F.Cu") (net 3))
 (segment (start 90.82 79.6556) (end 90.6483 79.8273) (width 0.2) (layer "F.Cu") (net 3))
 (via (at 107 92.514) (size 0.9) (drill 0.6) (layers "F.Cu" "B.Cu") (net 3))
 (segment (start 107 92.514) (end 107 94.294366) (width 0.2) (layer "B.Cu") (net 3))
 (segment (start 97.286 96.656) (end 104.638366 96.656) (width 0.2) (layer "B.Cu") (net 3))
 (segment (start 104.638366 96.656) (end 107 94.294366) (width 0.2) (layer "B.Cu") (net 3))
 (segment (start 96.135 95.505) (end 97.286 96.656) (width 0.2) (layer "B.Cu") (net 3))
 (segment (start 106.79 73.41) (end 105.2 75) (width 0.2) (layer "F.Cu") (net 11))
 (segment (start 105.2 75) (end 104 75) (width 0.2) (layer "F.Cu") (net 11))
 (via (at 104 75) (size 0.9) (drill 0.6) (layers "F.Cu" "B.Cu") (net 11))
 (segment (start 104 75) (end 104.251 74.749) (width 0.2) (layer "B.Cu") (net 11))
 (segment (start 104.251 74.749) (end 104.251 72.688925) (width 0.2) (layer "B.Cu") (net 11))
 (segment (start 104.251 72.688925) (end 101.667075 70.105) (width 0.2) (layer "B.Cu") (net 11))
 (segment (start 101.667075 70.105) (end 98.675 70.105) (width 0.2) (layer "B.Cu") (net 11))
 (segment (start 97.524 99.434) (end 98.675 100.585) (width 0.2) (layer "F.Cu") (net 5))
 (segment (start 106.79 58.17) (end 101.086 63.874) (width 0.2) (layer "F.Cu") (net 5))
 (segment (start 97.524 64.476) (end 97.524 99.434) (width 0.2) (layer "F.Cu") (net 5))
 (segment (start 101.086 63.874) (end 98.126 63.874) (width 0.2) (layer "F.Cu") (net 5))
 (segment (start 98.126 63.874) (end 97.524 64.476) (width 0.2) (layer "F.Cu") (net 5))
 (segment (start 110 66.46) (end 110 88.5) (width 0.2) (layer "F.Cu") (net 7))
 (segment (start 106.79 63.25) (end 110 66.46) (width 0.2) (layer "F.Cu") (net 7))
 (via (at 110 88.5) (size 0.9) (drill 0.6) (layers "F.Cu" "B.Cu") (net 7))
 (segment (start 105.68 88.5) (end 98.675 95.505) (width 0.2) (layer "B.Cu") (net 7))
 (segment (start 110 88.5) (end 105.68 88.5) (width 0.2) (layer "B.Cu") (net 7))
 (segment (start 106.79 70.87) (end 104.66 73) (width 0.2) (layer "F.Cu") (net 10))
 (segment (start 104.66 73) (end 103.5 73) (width 0.2) (layer "F.Cu") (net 10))
 (via (at 103.5 73) (size 0.9) (drill 0.6) (layers "F.Cu" "B.Cu") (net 10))
 (segment (start 103 73) (end 102.645 72.645) (width 0.2) (layer "B.Cu") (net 10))
 (segment (start 102.645 72.645) (end 98.675 72.645) (width 0.2) (layer "B.Cu") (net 10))
 (segment (start 103.5 73) (end 103 73) (width 0.2) (layer "B.Cu") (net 10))
 (segment (start 106.79 65.79) (end 101 71.58) (width 0.2) (layer "F.Cu") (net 8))
 (segment (start 101 71.58) (end 101 86.5) (width 0.2) (layer "F.Cu") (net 8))
 (via (at 101 86.5) (size 0.9) (drill 0.6) (layers "F.Cu" "B.Cu") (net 8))
 (segment (start 101 90.64) (end 98.675 92.965) (width 0.2) (layer "B.Cu") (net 8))
 (segment (start 101 86.5) (end 101 90.64) (width 0.2) (layer "B.Cu") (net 8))
 (segment (start 106.79 68.33) (end 101.75 73.37) (width 0.2) (layer "F.Cu") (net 9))
 (segment (start 101.75 73.37) (end 101.75 78) (width 0.2) (layer "F.Cu") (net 9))
 (via (at 101.75 78) (size 0.9) (drill 0.6) (layers "F.Cu" "B.Cu") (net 9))
 (segment (start 99.826 89.274) (end 98.675 90.425) (width 0.2) (layer "B.Cu") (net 9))
 (segment (start 99.826 79.924) (end 99.826 89.274) (width 0.2) (layer "B.Cu") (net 9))
 (segment (start 101.75 78) (end 99.826 79.924) (width 0.2) (layer "B.Cu") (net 9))
 (segment (start 91.7113 80.8903) (end 91.7113 77.0687) (width 0.2) (layer "F.Cu") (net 20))
 (segment (start 91.7113 77.0687) (end 96.135 72.645) (width 0.2) (layer "F.Cu") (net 20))
 (segment (start 89.23 106.77) (end 89.23 83.3716) (width 0.2) (layer "F.Cu") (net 20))
 (segment (start 89.23 83.3716) (end 91.7113 80.8903) (width 0.2) (layer "F.Cu") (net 20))
 (segment (start 100 96.72) (end 98.675 98.045) (width 0.2) (layer "F.Cu") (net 6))
 (segment (start 102.541634 91.764) (end 100 94.305634) (width 0.2) (layer "F.Cu") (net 6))
 (segment (start 100 94.305634) (end 100 96.72) (width 0.2) (layer "F.Cu") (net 6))
 (segment (start 115.071 90.813366) (end 114.120366 91.764) (width 0.2) (layer "F.Cu") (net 6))
 (segment (start 115.071 68.991) (end 115.071 90.813366) (width 0.2) (layer "F.Cu") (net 6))
 (segment (start 114.120366 91.764) (end 102.541634 91.764) (width 0.2) (layer "F.Cu") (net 6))
 (segment (start 106.79 60.71) (end 115.071 68.991) (width 0.2) (layer "F.Cu") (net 6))
 (segment (start 117.15 109.42) (end 103.4 95.67) (width 0.2) (layer "F.Cu") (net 36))
 (segment (start 117.15 114.05) (end 117.15 109.42) (width 0.2) (layer "F.Cu") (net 36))
 (segment (start 90.986793 109.801) (end 103.745999 109.801) (width 0.2) (layer "F.Cu") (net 34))
 (segment (start 87.96 105.5) (end 87.96 106.774207) (width 0.2) (layer "F.Cu") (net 34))
 (segment (start 87.96 106.774207) (end 90.986793 109.801) (width 0.2) (layer "F.Cu") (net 34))
 (segment (start 103.745999 109.801) (end 104.95 108.596999) (width 0.2) (layer "F.Cu") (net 34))
 (segment (start 104.95 108.596999) (end 104.95 102.05) (width 0.2) (layer "F.Cu") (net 34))
 (segment (start 90.6483 96.9723) (end 95.412 101.736) (width 0.2) (layer "F.Cu") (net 35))
 (segment (start 96.61176 101.736) (end 97.524 102.64824) (width 0.2) (layer "F.Cu") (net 35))
 (segment (start 97.524 104.64532) (end 100.87868 108) (width 0.2) (layer "F.Cu") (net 35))
 (segment (start 97.524 102.64824) (end 97.524 104.64532) (width 0.2) (layer "F.Cu") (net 35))
 (segment (start 100.87868 108) (end 103 108) (width 0.2) (layer "F.Cu") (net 35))
 (segment (start 95.412 101.736) (end 96.61176 101.736) (width 0.2) (layer "F.Cu") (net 35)))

